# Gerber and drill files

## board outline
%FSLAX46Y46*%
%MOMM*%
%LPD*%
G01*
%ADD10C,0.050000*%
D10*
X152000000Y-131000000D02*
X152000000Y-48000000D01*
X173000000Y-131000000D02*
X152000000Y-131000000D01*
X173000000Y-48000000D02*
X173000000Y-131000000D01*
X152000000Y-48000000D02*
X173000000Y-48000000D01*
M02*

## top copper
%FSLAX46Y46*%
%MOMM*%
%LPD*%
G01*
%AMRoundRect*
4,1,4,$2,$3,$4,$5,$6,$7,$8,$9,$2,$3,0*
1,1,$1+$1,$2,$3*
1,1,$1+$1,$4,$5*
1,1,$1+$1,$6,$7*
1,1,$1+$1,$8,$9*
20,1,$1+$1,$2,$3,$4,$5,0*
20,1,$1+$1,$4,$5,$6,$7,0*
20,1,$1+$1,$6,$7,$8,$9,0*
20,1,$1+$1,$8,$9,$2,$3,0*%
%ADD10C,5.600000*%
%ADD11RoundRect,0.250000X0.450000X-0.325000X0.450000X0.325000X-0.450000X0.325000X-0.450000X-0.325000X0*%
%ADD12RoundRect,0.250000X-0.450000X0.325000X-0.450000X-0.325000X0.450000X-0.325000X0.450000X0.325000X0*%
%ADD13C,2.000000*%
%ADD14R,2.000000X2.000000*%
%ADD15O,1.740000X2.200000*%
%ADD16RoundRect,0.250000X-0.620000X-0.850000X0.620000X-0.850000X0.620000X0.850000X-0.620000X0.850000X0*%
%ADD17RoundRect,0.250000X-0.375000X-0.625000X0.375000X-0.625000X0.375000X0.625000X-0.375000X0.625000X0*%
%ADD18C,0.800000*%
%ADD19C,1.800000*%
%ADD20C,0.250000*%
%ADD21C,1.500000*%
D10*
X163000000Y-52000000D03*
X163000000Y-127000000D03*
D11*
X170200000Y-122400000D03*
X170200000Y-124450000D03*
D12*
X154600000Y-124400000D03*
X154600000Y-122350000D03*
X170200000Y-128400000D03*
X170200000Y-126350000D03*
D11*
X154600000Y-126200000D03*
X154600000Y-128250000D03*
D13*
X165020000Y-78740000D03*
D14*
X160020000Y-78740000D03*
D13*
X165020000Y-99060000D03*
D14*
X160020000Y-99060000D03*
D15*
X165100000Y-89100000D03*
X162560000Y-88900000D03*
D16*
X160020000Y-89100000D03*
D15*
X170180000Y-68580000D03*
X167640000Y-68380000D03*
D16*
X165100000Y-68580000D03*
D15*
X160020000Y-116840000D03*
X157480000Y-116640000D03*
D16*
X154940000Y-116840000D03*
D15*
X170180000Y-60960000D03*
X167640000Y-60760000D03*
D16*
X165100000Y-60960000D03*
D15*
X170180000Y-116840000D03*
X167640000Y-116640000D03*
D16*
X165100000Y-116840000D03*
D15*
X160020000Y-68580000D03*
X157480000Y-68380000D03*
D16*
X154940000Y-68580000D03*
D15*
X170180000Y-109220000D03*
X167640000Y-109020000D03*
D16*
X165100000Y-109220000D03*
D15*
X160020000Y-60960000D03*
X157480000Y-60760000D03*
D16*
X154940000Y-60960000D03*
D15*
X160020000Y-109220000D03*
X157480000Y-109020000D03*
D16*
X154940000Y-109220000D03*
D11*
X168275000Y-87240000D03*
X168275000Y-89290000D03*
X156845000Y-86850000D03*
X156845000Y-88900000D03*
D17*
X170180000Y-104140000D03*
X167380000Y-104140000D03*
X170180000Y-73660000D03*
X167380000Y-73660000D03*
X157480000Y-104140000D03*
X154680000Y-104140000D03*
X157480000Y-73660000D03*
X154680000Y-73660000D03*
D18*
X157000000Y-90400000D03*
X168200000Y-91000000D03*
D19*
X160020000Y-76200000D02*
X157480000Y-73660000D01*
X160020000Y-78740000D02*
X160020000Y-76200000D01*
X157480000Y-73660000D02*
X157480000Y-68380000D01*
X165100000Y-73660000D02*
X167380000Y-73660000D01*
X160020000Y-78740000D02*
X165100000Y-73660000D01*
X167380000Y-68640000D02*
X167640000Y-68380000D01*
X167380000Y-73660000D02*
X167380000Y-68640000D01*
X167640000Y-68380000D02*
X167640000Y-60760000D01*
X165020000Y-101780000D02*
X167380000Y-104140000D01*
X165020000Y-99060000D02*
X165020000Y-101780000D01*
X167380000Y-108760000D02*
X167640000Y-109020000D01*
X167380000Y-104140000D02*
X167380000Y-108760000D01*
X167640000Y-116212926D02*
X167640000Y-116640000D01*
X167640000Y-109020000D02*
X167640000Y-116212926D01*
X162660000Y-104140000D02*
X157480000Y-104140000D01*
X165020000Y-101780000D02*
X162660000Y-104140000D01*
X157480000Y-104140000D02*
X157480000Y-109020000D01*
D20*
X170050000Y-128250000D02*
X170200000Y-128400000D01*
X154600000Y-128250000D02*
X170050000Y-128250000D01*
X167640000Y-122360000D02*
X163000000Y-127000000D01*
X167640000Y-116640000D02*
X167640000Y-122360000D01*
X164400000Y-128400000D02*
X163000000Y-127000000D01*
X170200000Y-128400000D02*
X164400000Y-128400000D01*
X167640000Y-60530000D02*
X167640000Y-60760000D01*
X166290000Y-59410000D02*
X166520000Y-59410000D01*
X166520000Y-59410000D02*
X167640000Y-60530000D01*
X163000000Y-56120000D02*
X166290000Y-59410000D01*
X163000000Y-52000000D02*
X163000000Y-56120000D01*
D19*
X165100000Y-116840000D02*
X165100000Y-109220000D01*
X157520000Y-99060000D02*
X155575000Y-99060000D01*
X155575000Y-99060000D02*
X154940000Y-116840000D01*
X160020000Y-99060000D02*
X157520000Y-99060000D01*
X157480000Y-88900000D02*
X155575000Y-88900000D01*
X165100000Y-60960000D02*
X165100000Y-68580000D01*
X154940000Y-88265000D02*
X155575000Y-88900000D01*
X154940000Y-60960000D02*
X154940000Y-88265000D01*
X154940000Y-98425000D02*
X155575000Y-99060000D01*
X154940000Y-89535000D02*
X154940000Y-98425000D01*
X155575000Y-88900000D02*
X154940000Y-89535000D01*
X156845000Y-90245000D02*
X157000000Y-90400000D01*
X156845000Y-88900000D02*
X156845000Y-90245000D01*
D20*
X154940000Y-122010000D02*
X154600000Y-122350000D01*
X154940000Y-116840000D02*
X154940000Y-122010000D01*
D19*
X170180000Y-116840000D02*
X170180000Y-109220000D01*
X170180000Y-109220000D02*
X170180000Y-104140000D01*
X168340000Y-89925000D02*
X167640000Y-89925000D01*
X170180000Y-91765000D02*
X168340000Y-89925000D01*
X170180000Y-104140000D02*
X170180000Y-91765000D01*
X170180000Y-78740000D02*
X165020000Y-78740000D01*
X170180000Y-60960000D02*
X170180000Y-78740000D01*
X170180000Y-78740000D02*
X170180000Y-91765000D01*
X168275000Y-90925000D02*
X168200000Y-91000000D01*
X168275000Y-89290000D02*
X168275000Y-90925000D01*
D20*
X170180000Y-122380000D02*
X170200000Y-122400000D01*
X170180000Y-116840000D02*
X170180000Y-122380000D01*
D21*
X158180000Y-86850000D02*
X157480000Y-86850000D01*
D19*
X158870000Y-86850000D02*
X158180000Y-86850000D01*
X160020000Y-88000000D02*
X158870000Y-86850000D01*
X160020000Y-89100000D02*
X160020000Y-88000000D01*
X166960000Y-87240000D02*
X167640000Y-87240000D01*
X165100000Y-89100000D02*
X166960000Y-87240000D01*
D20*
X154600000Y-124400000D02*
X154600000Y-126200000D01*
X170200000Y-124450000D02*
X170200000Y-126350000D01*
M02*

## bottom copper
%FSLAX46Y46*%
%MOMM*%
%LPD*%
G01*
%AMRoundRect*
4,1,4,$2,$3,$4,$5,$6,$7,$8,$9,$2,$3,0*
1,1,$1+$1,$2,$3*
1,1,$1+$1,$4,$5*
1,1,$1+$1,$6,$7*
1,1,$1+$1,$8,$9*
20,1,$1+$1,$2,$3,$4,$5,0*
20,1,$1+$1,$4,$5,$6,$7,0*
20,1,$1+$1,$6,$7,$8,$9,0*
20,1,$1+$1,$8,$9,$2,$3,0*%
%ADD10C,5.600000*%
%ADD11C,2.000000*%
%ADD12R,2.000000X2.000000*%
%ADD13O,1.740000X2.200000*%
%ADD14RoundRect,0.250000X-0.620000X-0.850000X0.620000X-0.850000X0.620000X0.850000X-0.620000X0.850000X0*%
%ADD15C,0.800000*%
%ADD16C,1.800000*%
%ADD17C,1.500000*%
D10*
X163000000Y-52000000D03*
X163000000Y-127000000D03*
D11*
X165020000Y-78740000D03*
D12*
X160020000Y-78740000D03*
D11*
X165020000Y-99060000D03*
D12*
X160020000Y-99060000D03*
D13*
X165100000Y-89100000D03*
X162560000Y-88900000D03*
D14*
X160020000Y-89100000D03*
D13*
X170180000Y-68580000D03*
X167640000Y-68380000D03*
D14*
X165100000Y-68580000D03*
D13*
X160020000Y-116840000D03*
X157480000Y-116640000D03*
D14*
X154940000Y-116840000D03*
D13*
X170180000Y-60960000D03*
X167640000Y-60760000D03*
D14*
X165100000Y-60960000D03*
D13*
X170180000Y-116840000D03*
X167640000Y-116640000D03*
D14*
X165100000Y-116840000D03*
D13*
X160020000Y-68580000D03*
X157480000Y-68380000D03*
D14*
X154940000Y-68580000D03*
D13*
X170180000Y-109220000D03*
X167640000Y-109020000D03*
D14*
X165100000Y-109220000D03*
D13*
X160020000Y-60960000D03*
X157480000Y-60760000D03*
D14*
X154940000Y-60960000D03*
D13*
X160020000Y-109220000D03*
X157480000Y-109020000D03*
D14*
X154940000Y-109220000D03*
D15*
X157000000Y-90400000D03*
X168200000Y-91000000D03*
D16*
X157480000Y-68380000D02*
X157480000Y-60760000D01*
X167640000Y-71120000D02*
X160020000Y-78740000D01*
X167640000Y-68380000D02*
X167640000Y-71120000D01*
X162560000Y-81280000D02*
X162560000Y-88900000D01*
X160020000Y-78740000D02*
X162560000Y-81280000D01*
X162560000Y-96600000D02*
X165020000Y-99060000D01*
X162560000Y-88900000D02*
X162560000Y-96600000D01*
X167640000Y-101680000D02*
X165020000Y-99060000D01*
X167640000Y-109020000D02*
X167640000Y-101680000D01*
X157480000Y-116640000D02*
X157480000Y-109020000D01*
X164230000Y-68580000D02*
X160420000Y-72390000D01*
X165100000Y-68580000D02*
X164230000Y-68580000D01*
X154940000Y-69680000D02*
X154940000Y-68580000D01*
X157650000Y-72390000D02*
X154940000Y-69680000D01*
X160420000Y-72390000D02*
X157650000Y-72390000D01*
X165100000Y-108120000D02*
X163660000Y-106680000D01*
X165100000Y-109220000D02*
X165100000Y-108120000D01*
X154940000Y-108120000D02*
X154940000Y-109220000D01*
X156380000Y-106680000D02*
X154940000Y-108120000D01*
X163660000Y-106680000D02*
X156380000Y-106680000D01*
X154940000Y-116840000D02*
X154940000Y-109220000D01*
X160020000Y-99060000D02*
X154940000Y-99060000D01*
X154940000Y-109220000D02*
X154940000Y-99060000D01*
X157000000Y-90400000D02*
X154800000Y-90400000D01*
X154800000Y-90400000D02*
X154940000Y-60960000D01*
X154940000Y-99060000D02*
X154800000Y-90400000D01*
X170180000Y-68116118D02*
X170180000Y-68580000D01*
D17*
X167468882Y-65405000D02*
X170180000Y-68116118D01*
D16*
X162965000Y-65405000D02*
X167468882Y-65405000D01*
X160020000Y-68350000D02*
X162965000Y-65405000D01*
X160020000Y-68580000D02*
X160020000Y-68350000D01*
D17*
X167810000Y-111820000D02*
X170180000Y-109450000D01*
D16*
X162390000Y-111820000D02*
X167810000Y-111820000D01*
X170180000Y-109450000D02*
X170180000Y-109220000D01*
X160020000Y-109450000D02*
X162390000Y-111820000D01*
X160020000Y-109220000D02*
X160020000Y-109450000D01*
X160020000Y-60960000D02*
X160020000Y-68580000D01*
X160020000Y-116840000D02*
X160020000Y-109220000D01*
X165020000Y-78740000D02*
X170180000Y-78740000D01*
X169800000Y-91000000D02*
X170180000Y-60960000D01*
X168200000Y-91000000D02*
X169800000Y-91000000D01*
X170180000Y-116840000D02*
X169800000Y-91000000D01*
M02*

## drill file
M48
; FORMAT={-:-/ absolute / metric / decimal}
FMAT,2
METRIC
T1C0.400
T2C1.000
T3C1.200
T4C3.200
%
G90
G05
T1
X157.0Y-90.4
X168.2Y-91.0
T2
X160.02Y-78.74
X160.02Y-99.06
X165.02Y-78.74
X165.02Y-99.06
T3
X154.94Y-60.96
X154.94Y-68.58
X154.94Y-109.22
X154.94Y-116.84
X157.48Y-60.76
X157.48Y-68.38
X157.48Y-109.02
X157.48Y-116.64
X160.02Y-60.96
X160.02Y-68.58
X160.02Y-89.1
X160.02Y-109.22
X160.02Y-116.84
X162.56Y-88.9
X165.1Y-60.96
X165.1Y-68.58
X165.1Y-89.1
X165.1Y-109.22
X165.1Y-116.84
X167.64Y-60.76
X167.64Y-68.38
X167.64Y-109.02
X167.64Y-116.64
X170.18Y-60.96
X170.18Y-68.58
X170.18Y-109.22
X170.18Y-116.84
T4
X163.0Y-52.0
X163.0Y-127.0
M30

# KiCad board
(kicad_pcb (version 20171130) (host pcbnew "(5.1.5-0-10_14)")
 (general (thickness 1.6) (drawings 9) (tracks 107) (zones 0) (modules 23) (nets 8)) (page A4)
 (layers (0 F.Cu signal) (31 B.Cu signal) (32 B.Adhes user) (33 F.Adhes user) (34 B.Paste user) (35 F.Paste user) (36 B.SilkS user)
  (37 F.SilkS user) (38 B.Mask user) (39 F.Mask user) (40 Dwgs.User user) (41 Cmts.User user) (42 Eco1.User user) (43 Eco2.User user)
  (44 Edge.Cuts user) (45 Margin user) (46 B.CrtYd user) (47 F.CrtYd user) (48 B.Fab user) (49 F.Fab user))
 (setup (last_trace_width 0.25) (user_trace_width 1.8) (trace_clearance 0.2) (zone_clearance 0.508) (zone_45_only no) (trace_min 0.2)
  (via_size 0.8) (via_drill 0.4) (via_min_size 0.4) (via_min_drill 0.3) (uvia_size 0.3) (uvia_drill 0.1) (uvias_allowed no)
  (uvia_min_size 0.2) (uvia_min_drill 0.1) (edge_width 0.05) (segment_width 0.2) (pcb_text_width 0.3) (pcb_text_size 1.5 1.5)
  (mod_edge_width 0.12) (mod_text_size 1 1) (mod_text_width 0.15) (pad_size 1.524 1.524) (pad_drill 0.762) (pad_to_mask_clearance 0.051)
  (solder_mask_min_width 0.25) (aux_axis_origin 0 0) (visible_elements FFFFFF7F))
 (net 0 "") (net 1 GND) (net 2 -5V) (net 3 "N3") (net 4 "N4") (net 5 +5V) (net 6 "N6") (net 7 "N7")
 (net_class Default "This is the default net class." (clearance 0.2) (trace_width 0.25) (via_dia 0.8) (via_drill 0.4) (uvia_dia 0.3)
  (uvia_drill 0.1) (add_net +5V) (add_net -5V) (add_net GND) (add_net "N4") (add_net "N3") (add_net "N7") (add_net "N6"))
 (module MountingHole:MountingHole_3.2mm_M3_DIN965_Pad (layer F.Cu) (at 163 52)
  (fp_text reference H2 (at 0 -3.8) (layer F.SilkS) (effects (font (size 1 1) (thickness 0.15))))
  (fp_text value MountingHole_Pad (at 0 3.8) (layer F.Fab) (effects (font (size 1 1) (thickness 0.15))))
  (pad 1 thru_hole circle (at 0 0) (size 5.6 5.6) (drill 3.2) (layers *.Cu *.Mask) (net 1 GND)))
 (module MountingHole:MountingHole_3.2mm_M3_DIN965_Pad (layer F.Cu) (at 163 127)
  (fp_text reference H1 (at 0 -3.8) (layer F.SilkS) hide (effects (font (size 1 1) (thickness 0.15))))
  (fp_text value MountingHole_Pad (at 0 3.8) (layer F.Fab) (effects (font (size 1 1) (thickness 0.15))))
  (pad 1 thru_hole circle (at 0 0) (size 5.6 5.6) (drill 3.2) (layers *.Cu *.Mask) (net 1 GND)))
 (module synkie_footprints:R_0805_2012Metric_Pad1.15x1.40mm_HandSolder (layer F.Cu) (at 170.2 123.425 90)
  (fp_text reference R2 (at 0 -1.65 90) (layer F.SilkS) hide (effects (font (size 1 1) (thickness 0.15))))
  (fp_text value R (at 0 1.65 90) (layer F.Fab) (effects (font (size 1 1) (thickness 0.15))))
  (pad 2 smd roundrect (at 1.025 0 90) (size 1.15 1.4) (layers F.Cu F.Paste F.Mask) (roundrect_rratio 0.217391) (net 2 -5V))
  (pad 1 smd roundrect (at -1.025 0 90) (size 1.15 1.4) (layers F.Cu F.Paste F.Mask) (roundrect_rratio 0.217391) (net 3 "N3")))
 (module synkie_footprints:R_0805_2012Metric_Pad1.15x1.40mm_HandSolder (layer F.Cu) (at 154.6 123.375 270)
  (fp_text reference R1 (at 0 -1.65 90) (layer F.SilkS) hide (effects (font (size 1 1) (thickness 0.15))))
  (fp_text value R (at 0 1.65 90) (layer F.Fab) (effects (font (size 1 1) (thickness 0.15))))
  (pad 2 smd roundrect (at 1.025 0 270) (size 1.15 1.4) (layers F.Cu F.Paste F.Mask) (roundrect_rratio 0.217391) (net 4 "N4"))
  (pad 1 smd roundrect (at -1.025 0 270) (size 1.15 1.4) (layers F.Cu F.Paste F.Mask) (roundrect_rratio 0.217391) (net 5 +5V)))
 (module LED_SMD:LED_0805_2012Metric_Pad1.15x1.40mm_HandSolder (layer F.Cu) (at 170.2 127.375 270)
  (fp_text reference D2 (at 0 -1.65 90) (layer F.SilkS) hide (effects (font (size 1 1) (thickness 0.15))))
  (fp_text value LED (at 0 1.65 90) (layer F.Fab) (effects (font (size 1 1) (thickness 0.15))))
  (pad 2 smd roundrect (at 1.025 0 270) (size 1.15 1.4) (layers F.Cu F.Paste F.Mask) (roundrect_rratio 0.217391) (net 1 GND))
  (pad 1 smd roundrect (at -1.025 0 270) (size 1.15 1.4) (layers F.Cu F.Paste F.Mask) (roundrect_rratio 0.217391) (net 3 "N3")))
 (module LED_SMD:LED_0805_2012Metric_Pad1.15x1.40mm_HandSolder (layer F.Cu) (at 154.6 127.225 90)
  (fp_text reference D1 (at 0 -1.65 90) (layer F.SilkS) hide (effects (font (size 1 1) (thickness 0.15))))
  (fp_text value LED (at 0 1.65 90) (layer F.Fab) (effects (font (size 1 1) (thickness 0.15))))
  (pad 2 smd roundrect (at 1.025 0 90) (size 1.15 1.4) (layers F.Cu F.Paste F.Mask) (roundrect_rratio 0.217391) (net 4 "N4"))
  (pad 1 smd roundrect (at -1.025 0 90) (size 1.15 1.4) (layers F.Cu F.Paste F.Mask) (roundrect_rratio 0.217391) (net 1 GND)))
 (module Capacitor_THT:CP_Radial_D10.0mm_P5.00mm (layer F.Cu) (at 160.02 78.74)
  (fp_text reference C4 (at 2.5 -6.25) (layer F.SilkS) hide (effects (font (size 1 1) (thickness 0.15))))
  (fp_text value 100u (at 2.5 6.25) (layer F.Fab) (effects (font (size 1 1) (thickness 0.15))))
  (pad 2 thru_hole circle (at 5 0) (size 2 2) (drill 1) (layers *.Cu *.Mask) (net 2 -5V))
  (pad 1 thru_hole rect (at 0 0) (size 2 2) (drill 1) (layers *.Cu *.Mask) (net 1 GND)))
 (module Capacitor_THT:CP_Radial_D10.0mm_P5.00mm (layer F.Cu) (at 160.02 99.06)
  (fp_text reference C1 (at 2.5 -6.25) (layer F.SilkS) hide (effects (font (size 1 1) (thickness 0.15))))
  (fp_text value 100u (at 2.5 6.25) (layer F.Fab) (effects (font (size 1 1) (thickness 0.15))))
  (pad 2 thru_hole circle (at 5 0) (size 2 2) (drill 1) (layers *.Cu *.Mask) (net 1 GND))
  (pad 1 thru_hole rect (at 0 0) (size 2 2) (drill 1) (layers *.Cu *.Mask) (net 5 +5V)))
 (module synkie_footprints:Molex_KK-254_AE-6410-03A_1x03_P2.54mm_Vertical (layer F.Cu) (at 160.02 89.1)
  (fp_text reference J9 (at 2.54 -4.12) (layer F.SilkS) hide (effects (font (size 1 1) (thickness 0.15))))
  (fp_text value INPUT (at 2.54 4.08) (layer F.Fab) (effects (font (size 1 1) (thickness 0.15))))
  (pad 3 thru_hole oval (at 5.08 0) (size 1.74 2.2) (drill 1.2) (layers *.Cu *.Mask) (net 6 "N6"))
  (pad 2 thru_hole oval (at 2.54 -0.2) (size 1.74 2.2) (drill 1.2) (layers *.Cu *.Mask) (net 1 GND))
  (pad 1 thru_hole roundrect (at 0 0) (size 1.74 2.2) (drill 1.2) (layers *.Cu *.Mask) (roundrect_rratio 0.143678) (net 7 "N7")))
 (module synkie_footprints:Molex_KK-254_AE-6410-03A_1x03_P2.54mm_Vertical (layer F.Cu) (at 165.1 68.58)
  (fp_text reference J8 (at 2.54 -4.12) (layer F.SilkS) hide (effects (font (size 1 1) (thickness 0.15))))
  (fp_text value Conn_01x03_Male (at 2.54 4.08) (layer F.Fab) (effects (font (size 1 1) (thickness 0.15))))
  (pad 3 thru_hole oval (at 5.08 0) (size 1.74 2.2) (drill 1.2) (layers *.Cu *.Mask) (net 2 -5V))
  (pad 2 thru_hole oval (at 2.54 -0.2) (size 1.74 2.2) (drill 1.2) (layers *.Cu *.Mask) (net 1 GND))
  (pad 1 thru_hole roundrect (at 0 0) (size 1.74 2.2) (drill 1.2) (layers *.Cu *.Mask) (roundrect_rratio 0.143678) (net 5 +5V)))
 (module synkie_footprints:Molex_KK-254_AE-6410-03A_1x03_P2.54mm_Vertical (layer F.Cu) (at 154.94 116.84)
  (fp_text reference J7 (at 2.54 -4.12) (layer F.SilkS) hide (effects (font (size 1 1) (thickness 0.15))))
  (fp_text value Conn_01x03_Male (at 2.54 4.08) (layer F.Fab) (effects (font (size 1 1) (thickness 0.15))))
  (pad 3 thru_hole oval (at 5.08 0) (size 1.74 2.2) (drill 1.2) (layers *.Cu *.Mask) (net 2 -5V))
  (pad 2 thru_hole oval (at 2.54 -0.2) (size 1.74 2.2) (drill 1.2) (layers *.Cu *.Mask) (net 1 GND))
  (pad 1 thru_hole roundrect (at 0 0) (size 1.74 2.2) (drill 1.2) (layers *.Cu *.Mask) (roundrect_rratio 0.143678) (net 5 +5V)))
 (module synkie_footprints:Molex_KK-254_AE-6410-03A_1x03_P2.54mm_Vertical (layer F.Cu) (at 165.1 60.96)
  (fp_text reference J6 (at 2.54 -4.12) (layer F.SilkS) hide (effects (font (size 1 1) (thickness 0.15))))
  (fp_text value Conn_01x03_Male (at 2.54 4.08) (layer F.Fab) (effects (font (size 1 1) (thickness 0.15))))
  (pad 3 thru_hole oval (at 5.08 0) (size 1.74 2.2) (drill 1.2) (layers *.Cu *.Mask) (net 2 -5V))
  (pad 2 thru_hole oval (at 2.54 -0.2) (size 1.74 2.2) (drill 1.2) (layers *.Cu *.Mask) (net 1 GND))
  (pad 1 thru_hole roundrect (at 0 0) (size 1.74 2.2) (drill 1.2) (layers *.Cu *.Mask) (roundrect_rratio 0.143678) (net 5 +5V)))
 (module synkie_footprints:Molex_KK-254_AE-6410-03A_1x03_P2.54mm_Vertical (layer F.Cu) (at 165.1 116.84)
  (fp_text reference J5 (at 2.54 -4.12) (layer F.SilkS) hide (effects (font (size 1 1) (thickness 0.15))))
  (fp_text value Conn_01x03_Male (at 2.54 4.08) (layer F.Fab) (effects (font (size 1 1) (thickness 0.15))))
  (pad 3 thru_hole oval (at 5.08 0) (size 1.74 2.2) (drill 1.2) (layers *.Cu *.Mask) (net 2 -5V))
  (pad 2 thru_hole oval (at 2.54 -0.2) (size 1.74 2.2) (drill 1.2) (layers *.Cu *.Mask) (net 1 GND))
  (pad 1 thru_hole roundrect (at 0 0) (size 1.74 2.2) (drill 1.2) (layers *.Cu *.Mask) (roundrect_rratio 0.143678) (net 5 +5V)))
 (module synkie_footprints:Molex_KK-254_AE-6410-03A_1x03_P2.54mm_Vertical (layer F.Cu) (at 154.94 68.58)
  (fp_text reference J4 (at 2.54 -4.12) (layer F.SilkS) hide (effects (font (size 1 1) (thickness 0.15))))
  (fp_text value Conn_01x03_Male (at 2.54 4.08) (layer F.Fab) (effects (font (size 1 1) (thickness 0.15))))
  (pad 3 thru_hole oval (at 5.08 0) (size 1.74 2.2) (drill 1.2) (layers *.Cu *.Mask) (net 2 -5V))
  (pad 2 thru_hole oval (at 2.54 -0.2) (size 1.74 2.2) (drill 1.2) (layers *.Cu *.Mask) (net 1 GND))
  (pad 1 thru_hole roundrect (at 0 0) (size 1.74 2.2) (drill 1.2) (layers *.Cu *.Mask) (roundrect_rratio 0.143678) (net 5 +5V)))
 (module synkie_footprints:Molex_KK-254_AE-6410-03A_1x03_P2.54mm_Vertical (layer F.Cu) (at 165.1 109.22)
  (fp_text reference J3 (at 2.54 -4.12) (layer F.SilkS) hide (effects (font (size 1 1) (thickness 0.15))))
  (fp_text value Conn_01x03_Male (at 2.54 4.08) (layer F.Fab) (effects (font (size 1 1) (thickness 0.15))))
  (pad 3 thru_hole oval (at 5.08 0) (size 1.74 2.2) (drill 1.2) (layers *.Cu *.Mask) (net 2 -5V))
  (pad 2 thru_hole oval (at 2.54 -0.2) (size 1.74 2.2) (drill 1.2) (layers *.Cu *.Mask) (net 1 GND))
  (pad 1 thru_hole roundrect (at 0 0) (size 1.74 2.2) (drill 1.2) (layers *.Cu *.Mask) (roundrect_rratio 0.143678) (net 5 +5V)))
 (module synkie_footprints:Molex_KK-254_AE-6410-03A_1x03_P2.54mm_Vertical (layer F.Cu) (at 154.94 60.96)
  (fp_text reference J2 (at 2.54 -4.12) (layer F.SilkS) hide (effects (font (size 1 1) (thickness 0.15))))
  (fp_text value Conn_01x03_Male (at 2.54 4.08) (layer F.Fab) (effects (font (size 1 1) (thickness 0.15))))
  (pad 3 thru_hole oval (at 5.08 0) (size 1.74 2.2) (drill 1.2) (layers *.Cu *.Mask) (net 2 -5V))
  (pad 2 thru_hole oval (at 2.54 -0.2) (size 1.74 2.2) (drill 1.2) (layers *.Cu *.Mask) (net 1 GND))
  (pad 1 thru_hole roundrect (at 0 0) (size 1.74 2.2) (drill 1.2) (layers *.Cu *.Mask) (roundrect_rratio 0.143678) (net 5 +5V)))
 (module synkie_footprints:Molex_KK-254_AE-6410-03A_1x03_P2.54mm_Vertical (layer F.Cu) (at 154.94 109.22)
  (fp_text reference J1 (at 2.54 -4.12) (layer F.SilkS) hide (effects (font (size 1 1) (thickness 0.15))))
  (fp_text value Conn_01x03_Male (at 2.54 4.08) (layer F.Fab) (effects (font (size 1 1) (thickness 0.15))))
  (pad 3 thru_hole oval (at 5.08 0) (size 1.74 2.2) (drill 1.2) (layers *.Cu *.Mask) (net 2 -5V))
  (pad 2 thru_hole oval (at 2.54 -0.2) (size 1.74 2.2) (drill 1.2) (layers *.Cu *.Mask) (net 1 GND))
  (pad 1 thru_hole roundrect (at 0 0) (size 1.74 2.2) (drill 1.2) (layers *.Cu *.Mask) (roundrect_rratio 0.143678) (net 5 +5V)))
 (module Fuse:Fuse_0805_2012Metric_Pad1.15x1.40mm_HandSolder (layer F.Cu) (at 168.275 88.265 90)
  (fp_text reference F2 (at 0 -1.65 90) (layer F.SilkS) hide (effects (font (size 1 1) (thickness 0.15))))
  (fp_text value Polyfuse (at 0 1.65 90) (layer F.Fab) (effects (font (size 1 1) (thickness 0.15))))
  (pad 2 smd roundrect (at 1.025 0 90) (size 1.15 1.4) (layers F.Cu F.Paste F.Mask) (roundrect_rratio 0.217391) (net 6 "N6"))
  (pad 1 smd roundrect (at -1.025 0 90) (size 1.15 1.4) (layers F.Cu F.Paste F.Mask) (roundrect_rratio 0.217391) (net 2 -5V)))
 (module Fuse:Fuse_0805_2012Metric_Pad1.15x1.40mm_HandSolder (layer F.Cu) (at 156.845 87.875 90)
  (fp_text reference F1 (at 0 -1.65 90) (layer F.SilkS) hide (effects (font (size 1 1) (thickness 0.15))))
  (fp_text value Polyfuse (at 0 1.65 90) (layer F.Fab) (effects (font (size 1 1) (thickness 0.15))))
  (pad 2 smd roundrect (at 1.025 0 90) (size 1.15 1.4) (layers F.Cu F.Paste F.Mask) (roundrect_rratio 0.217391) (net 7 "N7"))
  (pad 1 smd roundrect (at -1.025 0 90) (size 1.15 1.4) (layers F.Cu F.Paste F.Mask) (roundrect_rratio 0.217391) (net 5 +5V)))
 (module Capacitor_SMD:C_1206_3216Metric (layer F.Cu) (at 168.78 104.14)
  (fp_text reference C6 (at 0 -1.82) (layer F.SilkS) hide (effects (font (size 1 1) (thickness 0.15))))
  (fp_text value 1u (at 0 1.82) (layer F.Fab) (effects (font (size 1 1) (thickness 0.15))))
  (pad 2 smd roundrect (at 1.4 0) (size 1.25 1.75) (layers F.Cu F.Paste F.Mask) (roundrect_rratio 0.2) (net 2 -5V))
  (pad 1 smd roundrect (at -1.4 0) (size 1.25 1.75) (layers F.Cu F.Paste F.Mask) (roundrect_rratio 0.2) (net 1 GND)))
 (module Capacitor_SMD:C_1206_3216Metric (layer F.Cu) (at 168.78 73.66)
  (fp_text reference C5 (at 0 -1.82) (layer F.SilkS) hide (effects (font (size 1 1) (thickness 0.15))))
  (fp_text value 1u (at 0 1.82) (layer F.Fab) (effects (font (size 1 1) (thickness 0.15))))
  (pad 2 smd roundrect (at 1.4 0) (size 1.25 1.75) (layers F.Cu F.Paste F.Mask) (roundrect_rratio 0.2) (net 2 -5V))
  (pad 1 smd roundrect (at -1.4 0) (size 1.25 1.75) (layers F.Cu F.Paste F.Mask) (roundrect_rratio 0.2) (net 1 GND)))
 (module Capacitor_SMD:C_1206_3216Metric (layer F.Cu) (at 156.08 104.14)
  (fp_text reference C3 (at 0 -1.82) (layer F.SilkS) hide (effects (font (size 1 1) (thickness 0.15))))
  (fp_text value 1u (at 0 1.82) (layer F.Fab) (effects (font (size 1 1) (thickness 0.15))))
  (pad 2 smd roundrect (at 1.4 0) (size 1.25 1.75) (layers F.Cu F.Paste F.Mask) (roundrect_rratio 0.2) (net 1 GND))
  (pad 1 smd roundrect (at -1.4 0) (size 1.25 1.75) (layers F.Cu F.Paste F.Mask) (roundrect_rratio 0.2) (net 5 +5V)))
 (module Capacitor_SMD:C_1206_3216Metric (layer F.Cu) (at 156.08 73.66)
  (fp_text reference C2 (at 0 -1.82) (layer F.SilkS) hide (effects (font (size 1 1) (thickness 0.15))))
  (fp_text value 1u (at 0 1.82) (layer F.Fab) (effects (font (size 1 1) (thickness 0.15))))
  (pad 2 smd roundrect (at 1.4 0) (size 1.25 1.75) (layers F.Cu F.Paste F.Mask) (roundrect_rratio 0.2) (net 1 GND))
  (pad 1 smd roundrect (at -1.4 0) (size 1.25 1.75) (layers F.Cu F.Paste F.Mask) (roundrect_rratio 0.2) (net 5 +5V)))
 (gr_line (start 152 131) (end 152 48) (layer Edge.Cuts) (width 0.05))
 (gr_line (start 173 131) (end 152 131) (layer Edge.Cuts) (width 0.05))
 (gr_line (start 173 48) (end 173 131) (layer Edge.Cuts) (width 0.05))
 (gr_line (start 152 48) (end 173 48) (layer Edge.Cuts) (width 0.05))
 (segment (start 160.02 76.2) (end 157.48 73.66) (width 1.8) (layer F.Cu) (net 1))
 (segment (start 160.02 78.74) (end 160.02 76.2) (width 1.8) (layer F.Cu) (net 1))
 (segment (start 157.48 73.66) (end 157.48 68.38) (width 1.8) (layer F.Cu) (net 1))
 (segment (start 165.1 73.66) (end 167.38 73.66) (width 1.8) (layer F.Cu) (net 1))
 (segment (start 160.02 78.74) (end 165.1 73.66) (width 1.8) (layer F.Cu) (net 1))
 (segment (start 167.38 68.64) (end 167.64 68.38) (width 1.8) (layer F.Cu) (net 1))
 (segment (start 167.38 73.66) (end 167.38 68.64) (width 1.8) (layer F.Cu) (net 1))
 (segment (start 167.64 68.38) (end 167.64 60.76) (width 1.8) (layer F.Cu) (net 1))
 (segment (start 165.02 101.78) (end 167.38 104.14) (width 1.8) (layer F.Cu) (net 1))
 (segment (start 165.02 99.06) (end 165.02 101.78) (width 1.8) (layer F.Cu) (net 1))
 (segment (start 167.38 108.76) (end 167.64 109.02) (width 1.8) (layer F.Cu) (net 1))
 (segment (start 167.38 104.14) (end 167.38 108.76) (width 1.8) (layer F.Cu) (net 1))
 (segment (start 167.64 116.212926) (end 167.64 116.64) (width 1.8) (layer F.Cu) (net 1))
 (segment (start 167.64 109.02) (end 167.64 116.212926) (width 1.8) (layer F.Cu) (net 1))
 (segment (start 162.66 104.14) (end 157.48 104.14) (width 1.8) (layer F.Cu) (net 1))
 (segment (start 165.02 101.78) (end 162.66 104.14) (width 1.8) (layer F.Cu) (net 1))
 (segment (start 157.48 104.14) (end 157.48 109.02) (width 1.8) (layer F.Cu) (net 1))
 (segment (start 157.48 68.38) (end 157.48 60.76) (width 1.8) (layer B.Cu) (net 1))
 (segment (start 167.64 71.12) (end 160.02 78.74) (width 1.8) (layer B.Cu) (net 1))
 (segment (start 167.64 68.38) (end 167.64 71.12) (width 1.8) (layer B.Cu) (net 1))
 (segment (start 162.56 81.28) (end 162.56 88.9) (width 1.8) (layer B.Cu) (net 1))
 (segment (start 160.02 78.74) (end 162.56 81.28) (width 1.8) (layer B.Cu) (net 1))
 (segment (start 162.56 96.6) (end 165.02 99.06) (width 1.8) (layer B.Cu) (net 1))
 (segment (start 162.56 88.9) (end 162.56 96.6) (width 1.8) (layer B.Cu) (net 1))
 (segment (start 167.64 101.68) (end 165.02 99.06) (width 1.8) (layer B.Cu) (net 1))
 (segment (start 167.64 109.02) (end 167.64 101.68) (width 1.8) (layer B.Cu) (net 1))
 (segment (start 157.48 116.64) (end 157.48 109.02) (width 1.8) (layer B.Cu) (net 1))
 (segment (start 170.05 128.25) (end 170.2 128.4) (width 0.25) (layer F.Cu) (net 1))
 (segment (start 154.6 128.25) (end 170.05 128.25) (width 0.25) (layer F.Cu) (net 1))
 (segment (start 167.64 122.36) (end 163 127) (width 0.25) (layer F.Cu) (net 1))
 (segment (start 167.64 116.64) (end 167.64 122.36) (width 0.25) (layer F.Cu) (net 1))
 (segment (start 164.4 128.4) (end 163 127) (width 0.25) (layer F.Cu) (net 1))
 (segment (start 170.2 128.4) (end 164.4 128.4) (width 0.25) (layer F.Cu) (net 1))
 (segment (start 167.64 60.53) (end 167.64 60.76) (width 0.25) (layer F.Cu) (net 1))
 (segment (start 166.29 59.41) (end 166.52 59.41) (width 0.25) (layer F.Cu) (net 1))
 (segment (start 166.52 59.41) (end 167.64 60.53) (width 0.25) (layer F.Cu) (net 1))
 (segment (start 163 56.12) (end 166.29 59.41) (width 0.25) (layer F.Cu) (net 1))
 (segment (start 163 52) (end 163 56.12) (width 0.25) (layer F.Cu) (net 1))
 (segment (start 165.1 116.84) (end 165.1 109.22) (width 1.8) (layer F.Cu) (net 5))
 (segment (start 157.52 99.06) (end 155.575 99.06) (width 1.8) (layer F.Cu) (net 5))
 (segment (start 155.575 99.06) (end 154.94 116.84) (width 1.8) (layer F.Cu) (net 5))
 (segment (start 160.02 99.06) (end 157.52 99.06) (width 1.8) (layer F.Cu) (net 5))
 (segment (start 157.48 88.9) (end 155.575 88.9) (width 1.8) (layer F.Cu) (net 5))
 (segment (start 165.1 60.96) (end 165.1 68.58) (width 1.8) (layer F.Cu) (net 5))
 (segment (start 164.23 68.58) (end 160.42 72.39) (width 1.8) (layer B.Cu) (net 5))
 (segment (start 165.1 68.58) (end 164.23 68.58) (width 1.8) (layer B.Cu) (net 5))
 (segment (start 154.94 69.68) (end 154.94 68.58) (width 1.8) (layer B.Cu) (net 5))
 (segment (start 157.65 72.39) (end 154.94 69.68) (width 1.8) (layer B.Cu) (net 5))
 (segment (start 160.42 72.39) (end 157.65 72.39) (width 1.8) (layer B.Cu) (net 5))
 (segment (start 165.1 108.12) (end 163.66 106.68) (width 1.8) (layer B.Cu) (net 5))
 (segment (start 165.1 109.22) (end 165.1 108.12) (width 1.8) (layer B.Cu) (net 5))
 (segment (start 154.94 108.12) (end 154.94 109.22) (width 1.8) (layer B.Cu) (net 5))
 (segment (start 156.38 106.68) (end 154.94 108.12) (width 1.8) (layer B.Cu) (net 5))
 (segment (start 163.66 106.68) (end 156.38 106.68) (width 1.8) (layer B.Cu) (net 5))
 (segment (start 154.94 116.84) (end 154.94 109.22) (width 1.8) (layer B.Cu) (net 5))
 (segment (start 160.02 99.06) (end 154.94 99.06) (width 1.8) (layer B.Cu) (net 5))
 (segment (start 154.94 109.22) (end 154.94 99.06) (width 1.8) (layer B.Cu) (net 5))
 (segment (start 154.94 88.265) (end 155.575 88.9) (width 1.8) (layer F.Cu) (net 5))
 (segment (start 154.94 60.96) (end 154.94 88.265) (width 1.8) (layer F.Cu) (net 5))
 (segment (start 154.94 98.425) (end 155.575 99.06) (width 1.8) (layer F.Cu) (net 5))
 (segment (start 154.94 89.535) (end 154.94 98.425) (width 1.8) (layer F.Cu) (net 5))
 (segment (start 155.575 88.9) (end 154.94 89.535) (width 1.8) (layer F.Cu) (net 5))
 (via (at 157 90.4) (size 0.8) (drill 0.4) (layers F.Cu B.Cu) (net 5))
 (segment (start 156.845 90.245) (end 157 90.4) (width 1.8) (layer F.Cu) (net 5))
 (segment (start 156.845 88.9) (end 156.845 90.245) (width 1.8) (layer F.Cu) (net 5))
 (segment (start 157 90.4) (end 154.8 90.4) (width 1.8) (layer B.Cu) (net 5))
 (segment (start 154.8 90.4) (end 154.94 60.96) (width 1.8) (layer B.Cu) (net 5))
 (segment (start 154.94 99.06) (end 154.8 90.4) (width 1.8) (layer B.Cu) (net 5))
 (segment (start 154.94 122.01) (end 154.6 122.35) (width 0.25) (layer F.Cu) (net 5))
 (segment (start 154.94 116.84) (end 154.94 122.01) (width 0.25) (layer F.Cu) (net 5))
 (segment (start 170.18 116.84) (end 170.18 109.22) (width 1.8) (layer F.Cu) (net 2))
 (segment (start 170.18 109.22) (end 170.18 104.14) (width 1.8) (layer F.Cu) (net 2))
 (segment (start 168.34 89.925) (end 167.64 89.925) (width 1.8) (layer F.Cu) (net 2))
 (segment (start 170.18 91.765) (end 168.34 89.925) (width 1.8) (layer F.Cu) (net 2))
 (segment (start 170.18 104.14) (end 170.18 91.765) (width 1.8) (layer F.Cu) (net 2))
 (segment (start 170.18 78.74) (end 165.02 78.74) (width 1.8) (layer F.Cu) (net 2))
 (segment (start 170.18 60.96) (end 170.18 78.74) (width 1.8) (layer F.Cu) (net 2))
 (segment (start 170.18 68.116118) (end 170.18 68.58) (width 1.8) (layer B.Cu) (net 2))
 (segment (start 167.468882 65.405) (end 170.18 68.116118) (width 1.5) (layer B.Cu) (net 2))
 (segment (start 162.965 65.405) (end 167.468882 65.405) (width 1.8) (layer B.Cu) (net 2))
 (segment (start 160.02 68.35) (end 162.965 65.405) (width 1.8) (layer B.Cu) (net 2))
 (segment (start 160.02 68.58) (end 160.02 68.35) (width 1.8) (layer B.Cu) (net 2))
 (segment (start 167.81 111.82) (end 170.18 109.45) (width 1.5) (layer B.Cu) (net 2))
 (segment (start 162.39 111.82) (end 167.81 111.82) (width 1.8) (layer B.Cu) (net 2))
 (segment (start 170.18 109.45) (end 170.18 109.22) (width 1.8) (layer B.Cu) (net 2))
 (segment (start 160.02 109.45) (end 162.39 111.82) (width 1.8) (layer B.Cu) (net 2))
 (segment (start 160.02 109.22) (end 160.02 109.45) (width 1.8) (layer B.Cu) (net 2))
 (segment (start 160.02 60.96) (end 160.02 68.58) (width 1.8) (layer B.Cu) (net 2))
 (segment (start 160.02 116.84) (end 160.02 109.22) (width 1.8) (layer B.Cu) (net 2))
 (segment (start 165.02 78.74) (end 170.18 78.74) (width 1.8) (layer B.Cu) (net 2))
 (segment (start 170.18 78.74) (end 170.18 91.765) (width 1.8) (layer F.Cu) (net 2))
 (via (at 168.2 91) (size 0.8) (drill 0.4) (layers F.Cu B.Cu) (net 2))
 (segment (start 168.275 90.925) (end 168.2 91) (width 1.8) (layer F.Cu) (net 2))
 (segment (start 168.275 89.29) (end 168.275 90.925) (width 1.8) (layer F.Cu) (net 2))
 (segment (start 169.8 91) (end 170.18 60.96) (width 1.8) (layer B.Cu) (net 2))
 (segment (start 168.2 91) (end 169.8 91) (width 1.8) (layer B.Cu) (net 2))
 (segment (start 170.18 116.84) (end 169.8 91) (width 1.8) (layer B.Cu) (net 2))
 (segment (start 170.18 122.38) (end 170.2 122.4) (width 0.25) (layer F.Cu) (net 2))
 (segment (start 170.18 116.84) (end 170.18 122.38) (width 0.25) (layer F.Cu) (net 2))
 (segment (start 158.18 86.85) (end 157.48 86.85) (width 1.5) (layer F.Cu) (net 7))
 (segment (start 158.87 86.85) (end 158.18 86.85) (width 1.8) (layer F.Cu) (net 7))
 (segment (start 160.02 88) (end 158.87 86.85) (width 1.8) (layer F.Cu) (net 7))
 (segment (start 160.02 89.1) (end 160.02 88) (width 1.8) (layer F.Cu) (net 7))
 (segment (start 166.96 87.24) (end 167.64 87.24) (width 1.8) (layer F.Cu) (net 6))
 (segment (start 165.1 89.1) (end 166.96 87.24) (width 1.8) (layer F.Cu) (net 6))
 (segment (start 154.6 124.4) (end 154.6 126.2) (width 0.25) (layer F.Cu) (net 4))
 (segment (start 170.2 124.45) (end 170.2 126.35) (width 0.25) (layer F.Cu) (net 3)))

